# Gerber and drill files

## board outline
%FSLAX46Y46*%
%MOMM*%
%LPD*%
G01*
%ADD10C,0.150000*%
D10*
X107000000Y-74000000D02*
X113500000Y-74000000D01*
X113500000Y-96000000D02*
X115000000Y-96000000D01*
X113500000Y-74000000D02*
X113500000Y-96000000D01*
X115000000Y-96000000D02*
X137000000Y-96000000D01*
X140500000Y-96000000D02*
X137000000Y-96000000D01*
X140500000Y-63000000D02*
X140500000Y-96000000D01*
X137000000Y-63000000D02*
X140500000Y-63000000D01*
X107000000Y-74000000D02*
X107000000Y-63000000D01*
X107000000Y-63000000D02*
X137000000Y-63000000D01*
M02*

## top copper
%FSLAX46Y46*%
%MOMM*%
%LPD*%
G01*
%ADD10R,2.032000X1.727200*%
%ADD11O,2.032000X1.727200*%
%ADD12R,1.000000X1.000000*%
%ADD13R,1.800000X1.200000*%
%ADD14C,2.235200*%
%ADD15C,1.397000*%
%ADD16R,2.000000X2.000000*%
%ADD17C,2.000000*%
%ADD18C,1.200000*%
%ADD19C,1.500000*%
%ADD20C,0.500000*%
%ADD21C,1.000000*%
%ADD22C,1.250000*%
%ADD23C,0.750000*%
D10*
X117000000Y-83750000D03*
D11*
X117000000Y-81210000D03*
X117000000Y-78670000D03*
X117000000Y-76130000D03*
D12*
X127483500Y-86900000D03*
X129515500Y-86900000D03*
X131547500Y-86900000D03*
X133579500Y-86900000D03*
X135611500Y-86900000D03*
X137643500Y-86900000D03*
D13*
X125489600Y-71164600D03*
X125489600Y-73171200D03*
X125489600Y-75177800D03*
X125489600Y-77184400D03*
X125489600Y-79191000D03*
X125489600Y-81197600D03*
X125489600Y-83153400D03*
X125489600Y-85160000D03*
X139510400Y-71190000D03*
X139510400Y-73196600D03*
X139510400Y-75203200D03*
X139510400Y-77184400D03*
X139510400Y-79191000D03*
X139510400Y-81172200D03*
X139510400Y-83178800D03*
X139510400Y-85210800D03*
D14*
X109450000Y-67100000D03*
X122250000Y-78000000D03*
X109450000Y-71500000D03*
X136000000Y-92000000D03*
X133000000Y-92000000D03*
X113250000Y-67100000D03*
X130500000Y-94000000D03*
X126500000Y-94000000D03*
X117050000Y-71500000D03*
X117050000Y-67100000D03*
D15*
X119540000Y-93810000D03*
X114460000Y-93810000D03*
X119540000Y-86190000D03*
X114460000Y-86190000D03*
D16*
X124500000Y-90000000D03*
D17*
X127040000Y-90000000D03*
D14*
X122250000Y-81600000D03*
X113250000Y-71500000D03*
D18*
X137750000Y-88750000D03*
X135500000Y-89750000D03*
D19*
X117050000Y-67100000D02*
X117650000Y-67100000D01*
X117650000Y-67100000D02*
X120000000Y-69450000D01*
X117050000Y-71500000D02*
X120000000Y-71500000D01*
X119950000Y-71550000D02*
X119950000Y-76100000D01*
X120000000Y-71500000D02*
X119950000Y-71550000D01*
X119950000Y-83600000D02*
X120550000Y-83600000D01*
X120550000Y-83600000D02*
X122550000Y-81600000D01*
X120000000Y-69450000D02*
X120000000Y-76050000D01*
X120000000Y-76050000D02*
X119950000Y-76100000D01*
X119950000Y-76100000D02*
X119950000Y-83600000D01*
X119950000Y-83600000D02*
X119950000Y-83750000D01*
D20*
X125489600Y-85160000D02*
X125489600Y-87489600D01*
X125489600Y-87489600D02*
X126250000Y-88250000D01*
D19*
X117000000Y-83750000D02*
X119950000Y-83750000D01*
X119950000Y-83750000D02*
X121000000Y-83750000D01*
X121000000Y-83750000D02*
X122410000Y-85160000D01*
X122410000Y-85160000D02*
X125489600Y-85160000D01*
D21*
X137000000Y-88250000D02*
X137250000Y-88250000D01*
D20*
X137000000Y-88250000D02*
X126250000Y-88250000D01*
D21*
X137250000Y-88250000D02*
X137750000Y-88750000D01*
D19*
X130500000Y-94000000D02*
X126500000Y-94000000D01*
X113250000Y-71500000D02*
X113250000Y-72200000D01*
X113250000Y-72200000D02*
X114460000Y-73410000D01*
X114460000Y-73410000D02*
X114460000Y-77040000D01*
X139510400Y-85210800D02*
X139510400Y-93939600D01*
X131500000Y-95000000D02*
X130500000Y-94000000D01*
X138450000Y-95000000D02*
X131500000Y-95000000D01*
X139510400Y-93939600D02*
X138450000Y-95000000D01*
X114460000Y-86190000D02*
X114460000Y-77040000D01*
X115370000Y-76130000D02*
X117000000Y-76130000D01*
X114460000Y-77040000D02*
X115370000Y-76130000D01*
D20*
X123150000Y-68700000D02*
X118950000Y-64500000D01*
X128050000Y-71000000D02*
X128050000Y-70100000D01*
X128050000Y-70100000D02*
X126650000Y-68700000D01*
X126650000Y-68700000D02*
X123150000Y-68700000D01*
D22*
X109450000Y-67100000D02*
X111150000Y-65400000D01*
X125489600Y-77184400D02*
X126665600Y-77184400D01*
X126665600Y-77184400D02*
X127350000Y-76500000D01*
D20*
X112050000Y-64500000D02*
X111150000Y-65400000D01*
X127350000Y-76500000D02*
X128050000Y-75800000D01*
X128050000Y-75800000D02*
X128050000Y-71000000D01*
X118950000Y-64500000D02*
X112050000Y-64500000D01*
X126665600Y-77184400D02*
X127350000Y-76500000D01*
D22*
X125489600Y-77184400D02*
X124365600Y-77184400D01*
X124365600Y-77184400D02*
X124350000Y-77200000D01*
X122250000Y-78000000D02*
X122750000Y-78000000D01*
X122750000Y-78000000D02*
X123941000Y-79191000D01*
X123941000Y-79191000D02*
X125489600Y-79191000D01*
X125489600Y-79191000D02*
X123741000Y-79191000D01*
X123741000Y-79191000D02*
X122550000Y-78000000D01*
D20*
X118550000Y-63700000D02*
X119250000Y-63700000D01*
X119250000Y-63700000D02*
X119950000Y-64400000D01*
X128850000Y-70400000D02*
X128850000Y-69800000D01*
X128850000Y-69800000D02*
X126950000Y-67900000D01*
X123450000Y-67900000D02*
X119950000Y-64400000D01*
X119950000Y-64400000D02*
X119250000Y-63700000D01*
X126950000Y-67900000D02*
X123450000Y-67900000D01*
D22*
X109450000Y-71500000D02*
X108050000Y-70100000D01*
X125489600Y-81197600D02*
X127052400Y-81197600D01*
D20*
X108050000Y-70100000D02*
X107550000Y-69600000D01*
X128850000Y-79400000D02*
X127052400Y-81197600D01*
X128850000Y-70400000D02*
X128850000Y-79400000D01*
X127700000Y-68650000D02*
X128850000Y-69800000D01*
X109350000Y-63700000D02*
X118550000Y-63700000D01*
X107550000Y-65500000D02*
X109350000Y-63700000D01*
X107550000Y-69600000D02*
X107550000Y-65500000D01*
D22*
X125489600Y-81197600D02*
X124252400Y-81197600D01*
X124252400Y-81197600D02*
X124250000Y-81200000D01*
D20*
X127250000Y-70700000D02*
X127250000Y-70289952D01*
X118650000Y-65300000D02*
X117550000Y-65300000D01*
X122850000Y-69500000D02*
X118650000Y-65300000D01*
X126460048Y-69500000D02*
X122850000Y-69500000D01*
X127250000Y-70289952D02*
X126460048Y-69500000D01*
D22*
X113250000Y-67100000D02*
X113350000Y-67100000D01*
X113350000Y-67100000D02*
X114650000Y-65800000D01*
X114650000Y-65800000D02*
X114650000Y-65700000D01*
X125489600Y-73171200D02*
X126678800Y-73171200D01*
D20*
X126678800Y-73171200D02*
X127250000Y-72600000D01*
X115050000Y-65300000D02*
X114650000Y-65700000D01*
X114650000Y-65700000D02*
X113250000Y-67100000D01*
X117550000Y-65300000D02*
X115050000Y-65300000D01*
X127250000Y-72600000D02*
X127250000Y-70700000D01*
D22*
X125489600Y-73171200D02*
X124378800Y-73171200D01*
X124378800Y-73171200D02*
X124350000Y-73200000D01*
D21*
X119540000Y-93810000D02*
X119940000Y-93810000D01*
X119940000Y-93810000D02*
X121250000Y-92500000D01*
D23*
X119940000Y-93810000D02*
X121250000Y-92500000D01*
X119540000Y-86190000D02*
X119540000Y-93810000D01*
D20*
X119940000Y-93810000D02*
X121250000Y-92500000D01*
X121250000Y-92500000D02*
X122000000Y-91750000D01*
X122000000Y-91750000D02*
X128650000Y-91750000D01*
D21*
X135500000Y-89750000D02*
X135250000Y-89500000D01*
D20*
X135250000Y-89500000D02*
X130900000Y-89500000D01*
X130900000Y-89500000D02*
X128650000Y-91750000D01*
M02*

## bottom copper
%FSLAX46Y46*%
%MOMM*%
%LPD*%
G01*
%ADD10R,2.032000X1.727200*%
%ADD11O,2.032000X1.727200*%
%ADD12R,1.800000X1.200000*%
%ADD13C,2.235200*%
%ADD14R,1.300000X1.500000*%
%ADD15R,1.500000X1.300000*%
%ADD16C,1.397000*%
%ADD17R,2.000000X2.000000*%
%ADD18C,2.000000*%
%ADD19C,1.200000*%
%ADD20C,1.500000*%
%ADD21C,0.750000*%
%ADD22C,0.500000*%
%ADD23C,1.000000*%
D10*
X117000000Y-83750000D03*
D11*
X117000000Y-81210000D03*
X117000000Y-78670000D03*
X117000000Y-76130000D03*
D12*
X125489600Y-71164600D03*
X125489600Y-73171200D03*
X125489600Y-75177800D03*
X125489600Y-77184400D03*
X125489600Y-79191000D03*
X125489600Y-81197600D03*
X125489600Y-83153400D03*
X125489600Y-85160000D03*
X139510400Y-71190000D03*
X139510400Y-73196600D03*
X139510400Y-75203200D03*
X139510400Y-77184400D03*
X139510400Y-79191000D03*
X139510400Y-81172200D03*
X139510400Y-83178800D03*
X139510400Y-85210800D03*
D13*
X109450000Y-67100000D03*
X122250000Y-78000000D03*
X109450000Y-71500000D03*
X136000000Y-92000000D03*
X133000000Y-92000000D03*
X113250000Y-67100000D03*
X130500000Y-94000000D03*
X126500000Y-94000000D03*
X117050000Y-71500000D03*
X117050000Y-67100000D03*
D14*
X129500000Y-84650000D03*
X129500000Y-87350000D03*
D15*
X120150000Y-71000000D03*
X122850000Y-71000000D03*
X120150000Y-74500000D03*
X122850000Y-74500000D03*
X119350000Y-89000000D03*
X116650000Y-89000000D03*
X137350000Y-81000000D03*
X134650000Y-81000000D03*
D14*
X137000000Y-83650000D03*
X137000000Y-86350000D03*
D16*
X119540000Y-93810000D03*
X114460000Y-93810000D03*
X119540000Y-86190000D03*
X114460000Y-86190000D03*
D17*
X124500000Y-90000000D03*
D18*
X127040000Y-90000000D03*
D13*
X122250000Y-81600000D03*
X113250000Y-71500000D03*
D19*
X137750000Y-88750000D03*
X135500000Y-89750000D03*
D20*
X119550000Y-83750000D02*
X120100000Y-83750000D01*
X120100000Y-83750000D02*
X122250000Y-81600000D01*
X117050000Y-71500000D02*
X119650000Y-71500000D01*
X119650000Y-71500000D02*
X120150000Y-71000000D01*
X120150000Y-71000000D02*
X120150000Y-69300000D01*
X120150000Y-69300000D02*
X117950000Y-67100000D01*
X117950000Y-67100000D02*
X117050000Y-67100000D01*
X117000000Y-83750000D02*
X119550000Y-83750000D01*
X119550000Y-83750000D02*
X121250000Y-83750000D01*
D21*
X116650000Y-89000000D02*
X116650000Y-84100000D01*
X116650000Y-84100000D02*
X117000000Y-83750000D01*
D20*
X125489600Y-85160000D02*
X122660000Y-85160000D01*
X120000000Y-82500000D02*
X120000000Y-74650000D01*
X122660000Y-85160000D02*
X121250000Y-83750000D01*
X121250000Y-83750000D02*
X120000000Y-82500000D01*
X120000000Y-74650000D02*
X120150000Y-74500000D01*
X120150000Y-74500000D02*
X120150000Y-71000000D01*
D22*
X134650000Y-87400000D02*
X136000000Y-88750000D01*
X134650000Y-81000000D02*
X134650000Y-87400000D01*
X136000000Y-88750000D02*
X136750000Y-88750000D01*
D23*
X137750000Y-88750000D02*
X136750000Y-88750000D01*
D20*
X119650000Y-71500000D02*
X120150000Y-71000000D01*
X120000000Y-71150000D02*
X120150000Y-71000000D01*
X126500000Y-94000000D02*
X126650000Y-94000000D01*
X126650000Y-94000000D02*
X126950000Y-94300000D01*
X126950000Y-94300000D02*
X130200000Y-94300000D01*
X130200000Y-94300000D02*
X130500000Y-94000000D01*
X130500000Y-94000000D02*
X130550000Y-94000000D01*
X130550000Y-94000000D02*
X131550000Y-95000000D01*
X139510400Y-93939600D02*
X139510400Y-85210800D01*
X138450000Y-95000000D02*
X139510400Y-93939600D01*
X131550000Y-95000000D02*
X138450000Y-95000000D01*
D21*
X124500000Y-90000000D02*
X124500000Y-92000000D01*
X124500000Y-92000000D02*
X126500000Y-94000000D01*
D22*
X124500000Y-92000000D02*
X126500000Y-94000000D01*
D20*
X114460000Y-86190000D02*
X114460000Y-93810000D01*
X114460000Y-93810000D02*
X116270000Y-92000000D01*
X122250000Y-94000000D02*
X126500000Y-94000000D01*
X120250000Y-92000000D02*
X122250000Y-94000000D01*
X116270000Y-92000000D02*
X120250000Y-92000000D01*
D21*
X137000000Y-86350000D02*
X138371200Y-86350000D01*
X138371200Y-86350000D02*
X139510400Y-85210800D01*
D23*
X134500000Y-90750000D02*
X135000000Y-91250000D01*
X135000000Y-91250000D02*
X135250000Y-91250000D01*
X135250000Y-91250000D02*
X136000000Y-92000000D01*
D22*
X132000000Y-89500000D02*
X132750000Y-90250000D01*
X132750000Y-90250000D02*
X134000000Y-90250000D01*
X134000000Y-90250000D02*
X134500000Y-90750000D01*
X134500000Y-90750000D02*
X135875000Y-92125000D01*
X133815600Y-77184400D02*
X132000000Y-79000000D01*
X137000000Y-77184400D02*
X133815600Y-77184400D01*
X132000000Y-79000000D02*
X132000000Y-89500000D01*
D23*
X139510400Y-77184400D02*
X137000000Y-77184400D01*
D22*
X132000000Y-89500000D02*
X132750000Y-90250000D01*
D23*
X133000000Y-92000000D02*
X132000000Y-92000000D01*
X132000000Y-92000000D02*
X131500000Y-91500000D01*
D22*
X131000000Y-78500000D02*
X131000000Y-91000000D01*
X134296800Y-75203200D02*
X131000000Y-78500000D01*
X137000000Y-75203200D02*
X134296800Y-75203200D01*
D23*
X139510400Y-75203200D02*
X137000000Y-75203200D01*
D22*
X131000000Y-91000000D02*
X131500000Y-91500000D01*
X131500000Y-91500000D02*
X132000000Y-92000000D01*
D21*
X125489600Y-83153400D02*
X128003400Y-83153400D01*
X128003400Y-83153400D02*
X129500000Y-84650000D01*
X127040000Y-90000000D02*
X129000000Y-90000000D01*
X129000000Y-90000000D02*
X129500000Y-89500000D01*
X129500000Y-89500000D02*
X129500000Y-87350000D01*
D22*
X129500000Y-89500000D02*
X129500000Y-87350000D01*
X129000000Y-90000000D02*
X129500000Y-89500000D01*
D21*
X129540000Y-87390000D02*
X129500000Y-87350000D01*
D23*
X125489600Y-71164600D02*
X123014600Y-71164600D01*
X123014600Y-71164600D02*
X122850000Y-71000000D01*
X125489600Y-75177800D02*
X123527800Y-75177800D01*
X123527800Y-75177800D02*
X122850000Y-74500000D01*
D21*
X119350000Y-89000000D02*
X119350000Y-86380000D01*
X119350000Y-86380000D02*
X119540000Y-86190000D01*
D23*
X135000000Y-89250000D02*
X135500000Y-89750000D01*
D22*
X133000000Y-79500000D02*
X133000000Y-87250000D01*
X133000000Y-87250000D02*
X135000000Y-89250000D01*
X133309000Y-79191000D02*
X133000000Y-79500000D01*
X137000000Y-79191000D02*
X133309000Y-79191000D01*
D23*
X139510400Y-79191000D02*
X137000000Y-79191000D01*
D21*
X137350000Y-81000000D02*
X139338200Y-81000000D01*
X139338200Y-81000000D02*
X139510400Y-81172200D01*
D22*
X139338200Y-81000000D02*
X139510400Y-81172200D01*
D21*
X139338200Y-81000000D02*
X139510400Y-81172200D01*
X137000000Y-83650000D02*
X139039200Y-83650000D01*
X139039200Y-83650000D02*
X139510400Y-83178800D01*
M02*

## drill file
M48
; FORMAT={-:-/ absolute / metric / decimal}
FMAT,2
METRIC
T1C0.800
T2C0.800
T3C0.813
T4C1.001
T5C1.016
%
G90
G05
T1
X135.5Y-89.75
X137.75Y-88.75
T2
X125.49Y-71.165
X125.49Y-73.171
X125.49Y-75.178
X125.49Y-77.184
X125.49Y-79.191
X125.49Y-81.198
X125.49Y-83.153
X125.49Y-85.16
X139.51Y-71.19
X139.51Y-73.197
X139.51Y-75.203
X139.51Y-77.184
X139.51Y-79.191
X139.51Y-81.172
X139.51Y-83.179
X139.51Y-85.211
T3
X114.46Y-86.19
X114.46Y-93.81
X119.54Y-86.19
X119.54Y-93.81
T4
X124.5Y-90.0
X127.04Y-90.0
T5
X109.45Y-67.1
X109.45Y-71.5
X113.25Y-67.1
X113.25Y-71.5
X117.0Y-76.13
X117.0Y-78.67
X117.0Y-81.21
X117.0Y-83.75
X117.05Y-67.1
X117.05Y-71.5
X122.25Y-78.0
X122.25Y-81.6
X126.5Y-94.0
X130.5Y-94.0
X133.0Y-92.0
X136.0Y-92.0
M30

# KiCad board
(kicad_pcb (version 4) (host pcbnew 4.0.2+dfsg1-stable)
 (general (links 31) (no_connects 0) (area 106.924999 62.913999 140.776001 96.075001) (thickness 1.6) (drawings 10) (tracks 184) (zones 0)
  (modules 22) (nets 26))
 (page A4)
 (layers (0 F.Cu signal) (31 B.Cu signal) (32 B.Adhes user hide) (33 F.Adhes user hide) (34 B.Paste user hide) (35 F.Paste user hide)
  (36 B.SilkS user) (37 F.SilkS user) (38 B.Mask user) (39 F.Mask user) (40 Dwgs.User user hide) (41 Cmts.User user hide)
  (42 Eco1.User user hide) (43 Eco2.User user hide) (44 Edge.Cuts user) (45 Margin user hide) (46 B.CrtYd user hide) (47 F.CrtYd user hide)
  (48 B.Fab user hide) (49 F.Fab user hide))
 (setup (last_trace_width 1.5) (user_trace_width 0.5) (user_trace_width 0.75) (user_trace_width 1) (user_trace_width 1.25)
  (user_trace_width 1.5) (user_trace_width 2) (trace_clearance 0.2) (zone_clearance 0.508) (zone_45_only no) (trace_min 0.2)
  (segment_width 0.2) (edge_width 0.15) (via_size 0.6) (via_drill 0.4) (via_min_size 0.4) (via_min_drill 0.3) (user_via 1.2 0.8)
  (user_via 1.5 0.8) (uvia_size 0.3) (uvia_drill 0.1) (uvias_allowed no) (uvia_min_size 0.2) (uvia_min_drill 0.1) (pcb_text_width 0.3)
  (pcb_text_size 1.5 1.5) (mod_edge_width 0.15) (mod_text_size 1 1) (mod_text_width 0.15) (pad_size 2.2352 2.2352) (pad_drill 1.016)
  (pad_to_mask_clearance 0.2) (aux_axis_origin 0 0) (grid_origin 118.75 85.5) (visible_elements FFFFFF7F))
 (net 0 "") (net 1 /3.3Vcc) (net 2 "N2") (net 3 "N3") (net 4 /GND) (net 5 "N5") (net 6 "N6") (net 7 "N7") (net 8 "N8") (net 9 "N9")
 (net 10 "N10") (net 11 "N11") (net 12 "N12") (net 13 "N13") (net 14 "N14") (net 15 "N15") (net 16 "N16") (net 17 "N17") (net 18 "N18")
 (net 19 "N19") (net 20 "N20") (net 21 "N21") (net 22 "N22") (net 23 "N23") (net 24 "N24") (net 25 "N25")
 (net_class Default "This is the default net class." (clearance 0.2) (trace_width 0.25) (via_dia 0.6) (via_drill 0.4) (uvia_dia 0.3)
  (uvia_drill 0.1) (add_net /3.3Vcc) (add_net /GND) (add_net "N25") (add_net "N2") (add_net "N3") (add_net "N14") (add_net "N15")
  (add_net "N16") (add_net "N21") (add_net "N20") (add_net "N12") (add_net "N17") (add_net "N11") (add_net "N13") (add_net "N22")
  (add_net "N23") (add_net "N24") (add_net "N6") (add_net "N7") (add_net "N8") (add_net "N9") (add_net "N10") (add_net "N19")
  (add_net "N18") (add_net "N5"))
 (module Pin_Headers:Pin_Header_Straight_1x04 (layer F.Cu) (at 117 83.75 180)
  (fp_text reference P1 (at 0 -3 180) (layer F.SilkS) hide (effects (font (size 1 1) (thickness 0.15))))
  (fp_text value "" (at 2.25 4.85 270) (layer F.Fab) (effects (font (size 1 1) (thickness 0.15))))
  (pad 1 thru_hole rect (at 0 0 180) (size 2.032 1.7272) (drill 1.016) (layers *.Cu *.Mask F.SilkS) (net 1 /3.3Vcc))
  (pad 2 thru_hole oval (at 0 2.54 180) (size 2.032 1.7272) (drill 1.016) (layers *.Cu *.Mask F.SilkS) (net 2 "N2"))
  (pad 3 thru_hole oval (at 0 5.08 180) (size 2.032 1.7272) (drill 1.016) (layers *.Cu *.Mask F.SilkS) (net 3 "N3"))
  (pad 4 thru_hole oval (at 0 7.62 180) (size 2.032 1.7272) (drill 1.016) (layers *.Cu *.Mask F.SilkS) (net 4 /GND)))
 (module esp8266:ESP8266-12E (layer F.Cu) (at 132.5 75)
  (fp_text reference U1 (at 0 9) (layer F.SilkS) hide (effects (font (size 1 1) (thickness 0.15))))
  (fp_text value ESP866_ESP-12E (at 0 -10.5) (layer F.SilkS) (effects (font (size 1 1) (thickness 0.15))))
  (pad 9 smd rect (at -5.0165 11.9 90) (size 1 1) (layers F.Cu F.Paste F.Mask) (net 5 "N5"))
  (pad 10 smd rect (at -2.9845 11.9 90) (size 1 1) (layers F.Cu F.Paste F.Mask) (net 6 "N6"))
  (pad 11 smd rect (at -0.9525 11.9 90) (size 1 1) (layers F.Cu F.Paste F.Mask) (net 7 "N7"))
  (pad 12 smd rect (at 1.0795 11.9 90) (size 1 1) (layers F.Cu F.Paste F.Mask) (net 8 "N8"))
  (pad 13 smd rect (at 3.1115 11.9 90) (size 1 1) (layers F.Cu F.Paste F.Mask) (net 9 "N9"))
  (pad 14 smd rect (at 5.1435 11.9 90) (size 1 1) (layers F.Cu F.Paste F.Mask) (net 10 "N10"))
  (pad 1 thru_hole rect (at -7.0104 -3.8354) (size 1.8 1.2) (drill 0.8) (layers *.Cu *.Mask F.SilkS) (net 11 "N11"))
  (pad 2 thru_hole rect (at -7.0104 -1.8288) (size 1.8 1.2) (drill 0.8) (layers *.Cu *.Mask F.SilkS) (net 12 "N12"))
  (pad 3 thru_hole rect (at -7.0104 0.1778) (size 1.8 1.2) (drill 0.8) (layers *.Cu *.Mask F.SilkS) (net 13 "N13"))
  (pad 4 thru_hole rect (at -7.0104 2.1844) (size 1.8 1.2) (drill 0.8) (layers *.Cu *.Mask F.SilkS) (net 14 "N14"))
  (pad 5 thru_hole rect (at -7.0104 4.191) (size 1.8 1.2) (drill 0.8) (layers *.Cu *.Mask F.SilkS) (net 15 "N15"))
  (pad 6 thru_hole rect (at -7.0104 6.1976) (size 1.8 1.2) (drill 0.8) (layers *.Cu *.Mask F.SilkS) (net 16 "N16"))
  (pad 7 thru_hole rect (at -7.0104 8.1534) (size 1.8 1.2) (drill 0.8) (layers *.Cu *.Mask F.SilkS) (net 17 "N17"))
  (pad 8 thru_hole rect (at -7.0104 10.16) (size 1.8 1.2) (drill 0.8) (layers *.Cu *.Mask F.SilkS) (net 1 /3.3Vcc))
  (pad 22 thru_hole rect (at 7.0104 -3.81) (size 1.8 1.2) (drill 0.8) (layers *.Cu *.Mask F.SilkS) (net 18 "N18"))
  (pad 21 thru_hole rect (at 7.0104 -1.8034) (size 1.8 1.2) (drill 0.8) (layers *.Cu *.Mask F.SilkS) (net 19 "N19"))
  (pad 20 thru_hole rect (at 7.0104 0.2032) (size 1.8 1.2) (drill 0.8) (layers *.Cu *.Mask F.SilkS) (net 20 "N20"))
  (pad 19 thru_hole rect (at 7.0104 2.1844) (size 1.8 1.2) (drill 0.8) (layers *.Cu *.Mask F.SilkS) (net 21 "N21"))
  (pad 18 thru_hole rect (at 7.0104 4.191) (size 1.8 1.2) (drill 0.8) (layers *.Cu *.Mask F.SilkS) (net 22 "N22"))
  (pad 17 thru_hole rect (at 7.0104 6.1722) (size 1.8 1.2) (drill 0.8) (layers *.Cu *.Mask F.SilkS) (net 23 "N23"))
  (pad 16 thru_hole rect (at 7.0104 8.1788) (size 1.8 1.2) (drill 0.8) (layers *.Cu *.Mask F.SilkS) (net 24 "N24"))
  (pad 15 thru_hole rect (at 7.0104 10.2108) (size 1.8 1.2) (drill 0.8) (layers *.Cu *.Mask F.SilkS) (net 4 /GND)))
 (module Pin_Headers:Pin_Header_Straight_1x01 (layer F.Cu) (at 109.45 67.1)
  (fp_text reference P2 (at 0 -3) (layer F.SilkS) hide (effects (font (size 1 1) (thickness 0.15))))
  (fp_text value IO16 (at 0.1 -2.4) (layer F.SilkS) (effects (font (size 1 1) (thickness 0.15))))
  (pad 1 thru_hole circle (at 0 0) (size 2.2352 2.2352) (drill 1.016) (layers *.Cu *.Mask F.SilkS) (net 14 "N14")))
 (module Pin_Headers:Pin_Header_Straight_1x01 (layer F.Cu) (at 122.25 78)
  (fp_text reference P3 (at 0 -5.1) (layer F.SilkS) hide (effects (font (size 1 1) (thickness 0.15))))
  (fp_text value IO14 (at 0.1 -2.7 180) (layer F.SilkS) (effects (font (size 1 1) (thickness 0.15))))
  (pad 1 thru_hole circle (at 0 0) (size 2.2352 2.2352) (drill 1.016) (layers *.Cu *.Mask F.SilkS) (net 15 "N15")))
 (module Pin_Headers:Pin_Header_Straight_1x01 (layer F.Cu) (at 109.45 71.5)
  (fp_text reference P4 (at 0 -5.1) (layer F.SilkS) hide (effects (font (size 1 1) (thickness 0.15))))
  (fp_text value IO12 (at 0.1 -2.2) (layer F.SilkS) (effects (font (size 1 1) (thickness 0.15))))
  (pad 1 thru_hole circle (at 0 0) (size 2.2352 2.2352) (drill 1.016) (layers *.Cu *.Mask F.SilkS) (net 16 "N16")))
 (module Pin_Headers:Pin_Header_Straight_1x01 (layer F.Cu) (at 136 92)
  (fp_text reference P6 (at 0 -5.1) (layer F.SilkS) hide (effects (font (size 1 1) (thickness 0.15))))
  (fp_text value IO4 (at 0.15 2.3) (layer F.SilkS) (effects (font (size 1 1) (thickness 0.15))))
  (pad 1 thru_hole circle (at 0 0) (size 2.2352 2.2352) (drill 1.016) (layers *.Cu *.Mask F.SilkS) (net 21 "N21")))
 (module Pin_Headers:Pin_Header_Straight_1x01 (layer F.Cu) (at 133 92)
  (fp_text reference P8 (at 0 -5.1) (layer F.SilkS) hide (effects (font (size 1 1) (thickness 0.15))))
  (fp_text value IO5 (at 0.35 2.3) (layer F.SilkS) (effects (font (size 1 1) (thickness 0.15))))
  (pad 1 thru_hole circle (at 0 0) (size 2.2352 2.2352) (drill 1.016) (layers *.Cu *.Mask F.SilkS) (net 20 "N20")))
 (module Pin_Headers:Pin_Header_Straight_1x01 (layer F.Cu) (at 113.25 67.1)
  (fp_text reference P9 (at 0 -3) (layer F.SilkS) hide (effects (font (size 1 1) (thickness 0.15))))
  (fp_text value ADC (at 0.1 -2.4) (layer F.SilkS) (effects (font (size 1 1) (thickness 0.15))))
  (pad 1 thru_hole circle (at 0 0) (size 2.2352 2.2352) (drill 1.016) (layers *.Cu *.Mask F.SilkS) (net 12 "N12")))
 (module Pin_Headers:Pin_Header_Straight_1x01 (layer F.Cu) (at 130.5 94)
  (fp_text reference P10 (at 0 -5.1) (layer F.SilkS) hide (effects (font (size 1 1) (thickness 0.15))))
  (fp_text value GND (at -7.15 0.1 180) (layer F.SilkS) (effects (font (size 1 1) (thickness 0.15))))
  (pad 1 thru_hole circle (at 0 0) (size 2.2352 2.2352) (drill 1.016) (layers *.Cu *.Mask F.SilkS) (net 4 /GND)))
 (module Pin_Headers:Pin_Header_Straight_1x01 (layer F.Cu) (at 126.5 94)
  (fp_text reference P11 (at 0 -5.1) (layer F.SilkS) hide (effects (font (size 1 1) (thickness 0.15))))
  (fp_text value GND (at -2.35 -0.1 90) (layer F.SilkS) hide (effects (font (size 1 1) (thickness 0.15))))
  (pad 1 thru_hole circle (at 0 0) (size 2.2352 2.2352) (drill 1.016) (layers *.Cu *.Mask F.SilkS) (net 4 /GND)))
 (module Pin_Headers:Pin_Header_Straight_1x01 (layer F.Cu) (at 117.05 71.5)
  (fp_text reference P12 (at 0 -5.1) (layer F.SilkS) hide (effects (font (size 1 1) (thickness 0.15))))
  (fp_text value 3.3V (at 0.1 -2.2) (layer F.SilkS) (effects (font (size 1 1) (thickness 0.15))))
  (pad 1 thru_hole circle (at 0 0) (size 2.2352 2.2352) (drill 1.016) (layers *.Cu *.Mask F.SilkS) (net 1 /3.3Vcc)))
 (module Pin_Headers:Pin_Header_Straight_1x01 (layer F.Cu) (at 117.05 67.1)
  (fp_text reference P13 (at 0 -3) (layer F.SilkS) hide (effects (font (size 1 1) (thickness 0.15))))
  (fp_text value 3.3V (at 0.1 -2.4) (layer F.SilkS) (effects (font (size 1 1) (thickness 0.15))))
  (pad 1 thru_hole circle (at 0 0) (size 2.2352 2.2352) (drill 1.016) (layers *.Cu *.Mask F.SilkS) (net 1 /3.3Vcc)))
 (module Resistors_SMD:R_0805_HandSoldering (layer B.Cu) (at 129.5 86 270)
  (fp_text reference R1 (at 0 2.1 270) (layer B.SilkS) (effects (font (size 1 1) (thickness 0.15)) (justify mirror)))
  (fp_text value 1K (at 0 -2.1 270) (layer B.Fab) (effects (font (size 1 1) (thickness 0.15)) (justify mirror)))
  (pad 1 smd rect (at -1.35 0 270) (size 1.5 1.3) (layers B.Cu B.Paste B.Mask) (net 17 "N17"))
  (pad 2 smd rect (at 1.35 0 270) (size 1.5 1.3) (layers B.Cu B.Paste B.Mask) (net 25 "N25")))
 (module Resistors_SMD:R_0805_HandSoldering (layer B.Cu) (at 121.5 71)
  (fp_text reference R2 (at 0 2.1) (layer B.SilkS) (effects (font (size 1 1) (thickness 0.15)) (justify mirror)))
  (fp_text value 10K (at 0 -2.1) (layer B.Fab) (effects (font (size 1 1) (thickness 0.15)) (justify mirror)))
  (pad 1 smd rect (at -1.35 0) (size 1.5 1.3) (layers B.Cu B.Paste B.Mask) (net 1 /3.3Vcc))
  (pad 2 smd rect (at 1.35 0) (size 1.5 1.3) (layers B.Cu B.Paste B.Mask) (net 11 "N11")))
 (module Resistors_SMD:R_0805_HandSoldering (layer B.Cu) (at 121.5 74.5)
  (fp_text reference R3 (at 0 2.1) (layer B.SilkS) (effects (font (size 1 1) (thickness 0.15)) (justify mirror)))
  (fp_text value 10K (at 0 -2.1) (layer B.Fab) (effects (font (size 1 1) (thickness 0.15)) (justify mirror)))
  (pad 1 smd rect (at -1.35 0) (size 1.5 1.3) (layers B.Cu B.Paste B.Mask) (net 1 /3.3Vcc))
  (pad 2 smd rect (at 1.35 0) (size 1.5 1.3) (layers B.Cu B.Paste B.Mask) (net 13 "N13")))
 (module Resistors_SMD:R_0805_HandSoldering (layer B.Cu) (at 118 89 180)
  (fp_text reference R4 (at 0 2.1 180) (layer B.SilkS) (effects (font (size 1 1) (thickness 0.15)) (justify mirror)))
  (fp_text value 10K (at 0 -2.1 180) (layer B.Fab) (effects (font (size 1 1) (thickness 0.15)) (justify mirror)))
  (pad 1 smd rect (at -1.35 0 180) (size 1.5 1.3) (layers B.Cu B.Paste B.Mask) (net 22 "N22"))
  (pad 2 smd rect (at 1.35 0 180) (size 1.5 1.3) (layers B.Cu B.Paste B.Mask) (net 1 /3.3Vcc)))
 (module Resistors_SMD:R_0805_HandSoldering (layer B.Cu) (at 136 81 180)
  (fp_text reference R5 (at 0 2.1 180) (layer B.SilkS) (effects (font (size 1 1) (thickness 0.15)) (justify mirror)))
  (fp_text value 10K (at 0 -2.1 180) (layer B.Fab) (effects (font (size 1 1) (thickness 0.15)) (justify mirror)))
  (pad 1 smd rect (at -1.35 0 180) (size 1.5 1.3) (layers B.Cu B.Paste B.Mask) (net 23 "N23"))
  (pad 2 smd rect (at 1.35 0 180) (size 1.5 1.3) (layers B.Cu B.Paste B.Mask) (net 1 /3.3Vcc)))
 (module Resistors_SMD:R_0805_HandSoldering (layer B.Cu) (at 137 85 270)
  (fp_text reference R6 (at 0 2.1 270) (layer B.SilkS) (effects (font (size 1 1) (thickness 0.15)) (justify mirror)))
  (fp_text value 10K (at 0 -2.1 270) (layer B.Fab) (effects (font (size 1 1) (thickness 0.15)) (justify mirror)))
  (pad 1 smd rect (at -1.35 0 270) (size 1.5 1.3) (layers B.Cu B.Paste B.Mask) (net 24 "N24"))
  (pad 2 smd rect (at 1.35 0 270) (size 1.5 1.3) (layers B.Cu B.Paste B.Mask) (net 4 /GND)))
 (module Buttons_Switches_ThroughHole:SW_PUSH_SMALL (layer F.Cu) (at 117 90 270)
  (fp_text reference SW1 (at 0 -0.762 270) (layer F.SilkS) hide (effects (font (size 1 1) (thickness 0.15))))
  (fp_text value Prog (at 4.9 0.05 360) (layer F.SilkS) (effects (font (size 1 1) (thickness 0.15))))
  (pad 1 thru_hole circle (at 3.81 -2.54 270) (size 1.397 1.397) (drill 0.8128) (layers *.Cu *.Mask F.SilkS) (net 22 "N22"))
  (pad 2 thru_hole circle (at 3.81 2.54 270) (size 1.397 1.397) (drill 0.8128) (layers *.Cu *.Mask F.SilkS) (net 4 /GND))
  (pad 1 thru_hole circle (at -3.81 -2.54 270) (size 1.397 1.397) (drill 0.8128) (layers *.Cu *.Mask F.SilkS) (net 22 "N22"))
  (pad 2 thru_hole circle (at -3.81 2.54 270) (size 1.397 1.397) (drill 0.8128) (layers *.Cu *.Mask F.SilkS) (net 4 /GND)))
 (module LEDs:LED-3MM (layer F.Cu) (at 124.5 90)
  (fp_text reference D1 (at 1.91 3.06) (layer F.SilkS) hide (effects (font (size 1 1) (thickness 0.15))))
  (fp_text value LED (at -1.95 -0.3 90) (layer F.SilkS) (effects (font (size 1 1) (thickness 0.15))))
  (pad 1 thru_hole rect (at 0 0 90) (size 2 2) (drill 1.00076) (layers *.Cu *.Mask F.SilkS) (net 4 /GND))
  (pad 2 thru_hole circle (at 2.54 0) (size 2 2) (drill 1.00076) (layers *.Cu *.Mask F.SilkS) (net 25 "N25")))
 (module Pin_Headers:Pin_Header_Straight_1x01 (layer F.Cu) (at 122.25 81.6)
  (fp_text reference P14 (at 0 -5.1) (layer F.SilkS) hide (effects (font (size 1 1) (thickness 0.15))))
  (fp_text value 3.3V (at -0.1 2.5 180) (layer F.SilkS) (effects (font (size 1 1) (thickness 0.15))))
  (pad 1 thru_hole circle (at 0 0) (size 2.2352 2.2352) (drill 1.016) (layers *.Cu *.Mask F.SilkS) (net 1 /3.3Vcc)))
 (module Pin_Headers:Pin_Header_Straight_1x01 (layer F.Cu) (at 113.25 71.5)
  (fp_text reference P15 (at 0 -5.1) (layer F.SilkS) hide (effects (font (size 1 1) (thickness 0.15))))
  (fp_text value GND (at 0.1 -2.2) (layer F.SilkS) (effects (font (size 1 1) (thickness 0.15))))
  (pad 1 thru_hole circle (at 0 0) (size 2.2352 2.2352) (drill 1.016) (layers *.Cu *.Mask F.SilkS) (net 4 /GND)))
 (gr_line (start 107 74) (end 113.5 74) (angle 90) (layer Edge.Cuts) (width 0.15))
 (gr_line (start 113.5 96) (end 115 96) (angle 90) (layer Edge.Cuts) (width 0.15))
 (gr_line (start 113.5 74) (end 113.5 96) (angle 90) (layer Edge.Cuts) (width 0.15))
 (gr_line (start 115 96) (end 137 96) (angle 90) (layer Edge.Cuts) (width 0.15))
 (gr_line (start 140.5 96) (end 137 96) (angle 90) (layer Edge.Cuts) (width 0.15))
 (gr_line (start 140.5 63) (end 140.5 96) (angle 90) (layer Edge.Cuts) (width 0.15))
 (gr_line (start 137 63) (end 140.5 63) (angle 90) (layer Edge.Cuts) (width 0.15))
 (gr_line (start 107 74) (end 107 63) (angle 90) (layer Edge.Cuts) (width 0.15))
 (gr_line (start 107 63) (end 137 63) (angle 90) (layer Edge.Cuts) (width 0.15))
 (segment (start 119.55 83.75) (end 120.1 83.75) (width 1.5) (layer B.Cu) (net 1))
 (segment (start 120.1 83.75) (end 122.25 81.6) (width 1.5) (layer B.Cu) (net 1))
 (segment (start 117.05 71.5) (end 119.65 71.5) (width 1.5) (layer B.Cu) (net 1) (status 30))
 (segment (start 119.65 71.5) (end 120.15 71) (width 1.5) (layer B.Cu) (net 1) (status 30))
 (segment (start 120.15 71) (end 120.15 69.3) (width 1.5) (layer B.Cu) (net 1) (status 10))
 (segment (start 120.15 69.3) (end 117.95 67.1) (width 1.5) (layer B.Cu) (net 1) (status 20))
 (segment (start 117.95 67.1) (end 117.05 67.1) (width 1.5) (layer B.Cu) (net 1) (status 30))
 (segment (start 117.05 67.1) (end 117.65 67.1) (width 1.5) (layer F.Cu) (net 1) (status 30))
 (segment (start 117.65 67.1) (end 120 69.45) (width 1.5) (layer F.Cu) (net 1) (status 10))
 (segment (start 117.05 71.5) (end 120 71.5) (width 1.5) (layer F.Cu) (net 1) (status 10))
 (segment (start 119.95 71.55) (end 119.95 76.1) (width 1.5) (layer F.Cu) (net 1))
 (segment (start 120 71.5) (end 119.95 71.55) (width 1.5) (layer F.Cu) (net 1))
 (segment (start 119.95 83.6) (end 120.55 83.6) (width 1.5) (layer F.Cu) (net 1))
 (segment (start 120.55 83.6) (end 122.55 81.6) (width 1.5) (layer F.Cu) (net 1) (status 20))
 (segment (start 117 83.75) (end 119.55 83.75) (width 1.5) (layer B.Cu) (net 1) (status 10))
 (segment (start 119.55 83.75) (end 121.25 83.75) (width 1.5) (layer B.Cu) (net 1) (status 10))
 (segment (start 120 69.45) (end 120 76.05) (width 1.5) (layer F.Cu) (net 1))
 (segment (start 120 76.05) (end 119.95 76.1) (width 1.5) (layer F.Cu) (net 1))
 (segment (start 119.95 76.1) (end 119.95 83.6) (width 1.5) (layer F.Cu) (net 1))
 (segment (start 119.95 83.6) (end 119.95 83.75) (width 1.5) (layer F.Cu) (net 1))
 (segment (start 116.65 89) (end 116.65 84.1) (width 0.75) (layer B.Cu) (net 1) (status 30))
 (segment (start 116.65 84.1) (end 117 83.75) (width 0.75) (layer B.Cu) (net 1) (status 30))
 (segment (start 125.4896 85.16) (end 122.66 85.16) (width 1.5) (layer B.Cu) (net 1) (status 10))
 (segment (start 120 82.5) (end 120 74.65) (width 1.5) (layer B.Cu) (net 1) (status 20))
 (segment (start 122.66 85.16) (end 121.25 83.75) (width 1.5) (layer B.Cu) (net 1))
 (segment (start 121.25 83.75) (end 120 82.5) (width 1.5) (layer B.Cu) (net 1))
 (segment (start 120 74.65) (end 120.15 74.5) (width 1.5) (layer B.Cu) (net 1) (status 30))
 (segment (start 120.15 74.5) (end 120.15 71) (width 1.5) (layer B.Cu) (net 1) (status 30))
 (segment (start 125.4896 85.16) (end 125.4896 87.4896) (width 0.5) (layer F.Cu) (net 1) (status 10))
 (segment (start 125.4896 87.4896) (end 126.25 88.25) (width 0.5) (layer F.Cu) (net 1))
 (segment (start 117 83.75) (end 119.95 83.75) (width 1.5) (layer F.Cu) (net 1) (status 10))
 (segment (start 119.95 83.75) (end 121 83.75) (width 1.5) (layer F.Cu) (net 1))
 (segment (start 121 83.75) (end 122.41 85.16) (width 1.5) (layer F.Cu) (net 1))
 (segment (start 122.41 85.16) (end 125.4896 85.16) (width 1.5) (layer F.Cu) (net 1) (status 20))
 (segment (start 137 88.25) (end 137.25 88.25) (width 1) (layer F.Cu) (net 1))
 (segment (start 137 88.25) (end 126.25 88.25) (width 0.5) (layer F.Cu) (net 1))
 (segment (start 134.65 87.4) (end 136 88.75) (width 0.5) (layer B.Cu) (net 1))
 (segment (start 134.65 81) (end 134.65 87.4) (width 0.5) (layer B.Cu) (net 1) (status 10))
 (segment (start 136 88.75) (end 136.75 88.75) (width 0.5) (layer B.Cu) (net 1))
 (via (at 137.75 88.75) (size 1.2) (drill 0.8) (layers F.Cu B.Cu) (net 1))
 (segment (start 137.75 88.75) (end 136.75 88.75) (width 1) (layer B.Cu) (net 1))
 (segment (start 137.25 88.25) (end 137.75 88.75) (width 1) (layer F.Cu) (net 1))
 (segment (start 119.65 71.5) (end 120.15 71) (width 1.5) (layer B.Cu) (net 1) (status 30))
 (segment (start 120 71.15) (end 120.15 71) (width 1.5) (layer B.Cu) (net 1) (status 30))
 (segment (start 126.5 94) (end 126.65 94) (width 1.5) (layer B.Cu) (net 4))
 (segment (start 126.65 94) (end 126.95 94.3) (width 1.5) (layer B.Cu) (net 4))
 (segment (start 126.95 94.3) (end 130.2 94.3) (width 1.5) (layer B.Cu) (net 4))
 (segment (start 130.2 94.3) (end 130.5 94) (width 1.5) (layer B.Cu) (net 4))
 (segment (start 130.5 94) (end 126.5 94) (width 1.5) (layer F.Cu) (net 4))
 (segment (start 113.25 71.5) (end 113.25 72.2) (width 1.5) (layer F.Cu) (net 4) (status 30))
 (segment (start 113.25 72.2) (end 114.46 73.41) (width 1.5) (layer F.Cu) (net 4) (status 10))
 (segment (start 114.46 73.41) (end 114.46 77.04) (width 1.5) (layer F.Cu) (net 4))
 (segment (start 130.5 94) (end 130.55 94) (width 1.5) (layer B.Cu) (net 4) (status 30))
 (segment (start 130.55 94) (end 131.55 95) (width 1.5) (layer B.Cu) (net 4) (status 10))
 (segment (start 139.5104 93.9396) (end 139.5104 85.2108) (width 1.5) (layer B.Cu) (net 4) (status 20))
 (segment (start 138.45 95) (end 139.5104 93.9396) (width 1.5) (layer B.Cu) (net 4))
 (segment (start 131.55 95) (end 138.45 95) (width 1.5) (layer B.Cu) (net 4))
 (segment (start 139.5104 85.2108) (end 139.5104 93.9396) (width 1.5) (layer F.Cu) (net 4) (status 10))
 (segment (start 131.5 95) (end 130.5 94) (width 1.5) (layer F.Cu) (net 4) (status 20))
 (segment (start 138.45 95) (end 131.5 95) (width 1.5) (layer F.Cu) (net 4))
 (segment (start 139.5104 93.9396) (end 138.45 95) (width 1.5) (layer F.Cu) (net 4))
 (segment (start 124.5 90) (end 124.5 92) (width 0.75) (layer B.Cu) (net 4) (status 10))
 (segment (start 124.5 92) (end 126.5 94) (width 0.75) (layer B.Cu) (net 4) (status 20))
 (segment (start 124.5 92) (end 126.5 94) (width 0.5) (layer B.Cu) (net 4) (status 20))
 (segment (start 114.46 86.19) (end 114.46 93.81) (width 1.5) (layer B.Cu) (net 4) (status 30))
 (segment (start 114.46 93.81) (end 116.27 92) (width 1.5) (layer B.Cu) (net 4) (status 10))
 (segment (start 122.25 94) (end 126.5 94) (width 1.5) (layer B.Cu) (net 4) (status 20))
 (segment (start 120.25 92) (end 122.25 94) (width 1.5) (layer B.Cu) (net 4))
 (segment (start 116.27 92) (end 120.25 92) (width 1.5) (layer B.Cu) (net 4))
 (segment (start 114.46 86.19) (end 114.46 77.04) (width 1.5) (layer F.Cu) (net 4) (status 10))
 (segment (start 115.37 76.13) (end 117 76.13) (width 1.5) (layer F.Cu) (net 4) (status 20))
 (segment (start 114.46 77.04) (end 115.37 76.13) (width 1.5) (layer F.Cu) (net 4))
 (segment (start 137 86.35) (end 138.3712 86.35) (width 0.75) (layer B.Cu) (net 4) (status 10))
 (segment (start 138.3712 86.35) (end 139.5104 85.2108) (width 0.75) (layer B.Cu) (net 4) (status 20))
 (segment (start 123.15 68.7) (end 118.95 64.5) (width 0.5) (layer F.Cu) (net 14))
 (segment (start 128.05 71) (end 128.05 70.1) (width 0.5) (layer F.Cu) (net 14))
 (segment (start 128.05 70.1) (end 126.65 68.7) (width 0.5) (layer F.Cu) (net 14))
 (segment (start 126.65 68.7) (end 123.15 68.7) (width 0.5) (layer F.Cu) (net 14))
 (segment (start 109.45 67.1) (end 111.15 65.4) (width 1.25) (layer F.Cu) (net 14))
 (segment (start 125.4896 77.1844) (end 126.6656 77.1844) (width 1.25) (layer F.Cu) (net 14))
 (segment (start 126.6656 77.1844) (end 127.35 76.5) (width 1.25) (layer F.Cu) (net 14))
 (segment (start 112.05 64.5) (end 111.15 65.4) (width 0.5) (layer F.Cu) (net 14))
 (segment (start 127.35 76.5) (end 128.05 75.8) (width 0.5) (layer F.Cu) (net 14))
 (segment (start 128.05 75.8) (end 128.05 71) (width 0.5) (layer F.Cu) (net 14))
 (segment (start 118.95 64.5) (end 112.05 64.5) (width 0.5) (layer F.Cu) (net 14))
 (segment (start 126.6656 77.1844) (end 127.35 76.5) (width 0.5) (layer F.Cu) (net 14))
 (segment (start 125.4896 77.1844) (end 124.3656 77.1844) (width 1.25) (layer F.Cu) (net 14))
 (segment (start 124.3656 77.1844) (end 124.35 77.2) (width 1.25) (layer F.Cu) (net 14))
 (segment (start 122.25 78) (end 122.75 78) (width 1.25) (layer F.Cu) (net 15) (status 30))
 (segment (start 122.75 78) (end 123.941 79.191) (width 1.25) (layer F.Cu) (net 15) (status 10))
 (segment (start 123.941 79.191) (end 125.4896 79.191) (width 1.25) (layer F.Cu) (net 15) (status 20))
 (segment (start 125.4896 79.191) (end 123.741 79.191) (width 1.25) (layer F.Cu) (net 15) (status 10))
 (segment (start 123.741 79.191) (end 122.55 78) (width 1.25) (layer F.Cu) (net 15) (status 20))
 (segment (start 118.55 63.7) (end 119.25 63.7) (width 0.5) (layer F.Cu) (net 16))
 (segment (start 119.25 63.7) (end 119.95 64.4) (width 0.5) (layer F.Cu) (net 16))
 (segment (start 128.85 70.4) (end 128.85 69.8) (width 0.5) (layer F.Cu) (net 16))
 (segment (start 128.85 69.8) (end 126.95 67.9) (width 0.5) (layer F.Cu) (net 16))
 (segment (start 123.45 67.9) (end 119.95 64.4) (width 0.5) (layer F.Cu) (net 16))
 (segment (start 119.95 64.4) (end 119.25 63.7) (width 0.5) (layer F.Cu) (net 16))
 (segment (start 126.95 67.9) (end 123.45 67.9) (width 0.5) (layer F.Cu) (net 16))
 (segment (start 109.45 71.5) (end 108.05 70.1) (width 1.25) (layer F.Cu) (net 16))
 (segment (start 125.4896 81.1976) (end 127.0524 81.1976) (width 1.25) (layer F.Cu) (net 16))
 (segment (start 108.05 70.1) (end 107.55 69.6) (width 0.5) (layer F.Cu) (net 16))
 (segment (start 128.85 79.4) (end 127.0524 81.1976) (width 0.5) (layer F.Cu) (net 16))
 (segment (start 128.85 70.4) (end 128.85 79.4) (width 0.5) (layer F.Cu) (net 16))
 (segment (start 127.7 68.65) (end 128.85 69.8) (width 0.5) (layer F.Cu) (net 16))
 (segment (start 109.35 63.7) (end 118.55 63.7) (width 0.5) (layer F.Cu) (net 16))
 (segment (start 107.55 65.5) (end 109.35 63.7) (width 0.5) (layer F.Cu) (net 16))
 (segment (start 107.55 69.6) (end 107.55 65.5) (width 0.5) (layer F.Cu) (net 16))
 (segment (start 125.4896 81.1976) (end 124.2524 81.1976) (width 1.25) (layer F.Cu) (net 16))
 (segment (start 124.2524 81.1976) (end 124.25 81.2) (width 1.25) (layer F.Cu) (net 16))
 (segment (start 134.5 90.75) (end 135 91.25) (width 1) (layer B.Cu) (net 21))
 (segment (start 135 91.25) (end 135.25 91.25) (width 1) (layer B.Cu) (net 21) (status 20))
 (segment (start 135.25 91.25) (end 136 92) (width 1) (layer B.Cu) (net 21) (status 30))
 (segment (start 132 89.5) (end 132.75 90.25) (width 0.5) (layer B.Cu) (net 21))
 (segment (start 132.75 90.25) (end 134 90.25) (width 0.5) (layer B.Cu) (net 21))
 (segment (start 134 90.25) (end 134.5 90.75) (width 0.5) (layer B.Cu) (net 21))
 (segment (start 134.5 90.75) (end 135.875 92.125) (width 0.5) (layer B.Cu) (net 21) (status 20))
 (segment (start 133.8156 77.1844) (end 132 79) (width 0.5) (layer B.Cu) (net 21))
 (segment (start 137 77.1844) (end 133.8156 77.1844) (width 0.5) (layer B.Cu) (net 21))
 (segment (start 132 79) (end 132 89.5) (width 0.5) (layer B.Cu) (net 21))
 (segment (start 139.5104 77.1844) (end 137 77.1844) (width 1) (layer B.Cu) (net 21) (status 10))
 (segment (start 132 89.5) (end 132.75 90.25) (width 0.5) (layer B.Cu) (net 21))
 (segment (start 133 92) (end 132 92) (width 1) (layer B.Cu) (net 20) (status 30))
 (segment (start 132 92) (end 131.5 91.5) (width 1) (layer B.Cu) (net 20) (status 10))
 (segment (start 131 78.5) (end 131 91) (width 0.5) (layer B.Cu) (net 20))
 (segment (start 134.2968 75.2032) (end 131 78.5) (width 0.5) (layer B.Cu) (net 20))
 (segment (start 137 75.2032) (end 134.2968 75.2032) (width 0.5) (layer B.Cu) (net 20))
 (segment (start 139.5104 75.2032) (end 137 75.2032) (width 1) (layer B.Cu) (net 20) (status 10))
 (segment (start 131 91) (end 131.5 91.5) (width 0.5) (layer B.Cu) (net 20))
 (segment (start 131.5 91.5) (end 132 92) (width 0.5) (layer B.Cu) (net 20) (status 20))
 (segment (start 127.25 70.7) (end 127.25 70.289952) (width 0.5) (layer F.Cu) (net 12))
 (segment (start 118.65 65.3) (end 117.55 65.3) (width 0.5) (layer F.Cu) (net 12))
 (segment (start 122.85 69.5) (end 118.65 65.3) (width 0.5) (layer F.Cu) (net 12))
 (segment (start 126.460048 69.5) (end 122.85 69.5) (width 0.5) (layer F.Cu) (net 12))
 (segment (start 127.25 70.289952) (end 126.460048 69.5) (width 0.5) (layer F.Cu) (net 12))
 (segment (start 113.25 67.1) (end 113.35 67.1) (width 1.25) (layer F.Cu) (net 12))
 (segment (start 113.35 67.1) (end 114.65 65.8) (width 1.25) (layer F.Cu) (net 12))
 (segment (start 114.65 65.8) (end 114.65 65.7) (width 1.25) (layer F.Cu) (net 12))
 (segment (start 125.4896 73.1712) (end 126.6788 73.1712) (width 1.25) (layer F.Cu) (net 12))
 (segment (start 126.6788 73.1712) (end 127.25 72.6) (width 0.5) (layer F.Cu) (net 12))
 (segment (start 115.05 65.3) (end 114.65 65.7) (width 0.5) (layer F.Cu) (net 12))
 (segment (start 114.65 65.7) (end 113.25 67.1) (width 0.5) (layer F.Cu) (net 12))
 (segment (start 117.55 65.3) (end 115.05 65.3) (width 0.5) (layer F.Cu) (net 12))
 (segment (start 127.25 72.6) (end 127.25 70.7) (width 0.5) (layer F.Cu) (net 12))
 (segment (start 125.4896 73.1712) (end 124.3788 73.1712) (width 1.25) (layer F.Cu) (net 12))
 (segment (start 124.3788 73.1712) (end 124.35 73.2) (width 1.25) (layer F.Cu) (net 12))
 (segment (start 125.4896 83.1534) (end 128.0034 83.1534) (width 0.75) (layer B.Cu) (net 17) (status 10))
 (segment (start 128.0034 83.1534) (end 129.5 84.65) (width 0.75) (layer B.Cu) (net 17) (status 20))
 (segment (start 127.04 90) (end 129 90) (width 0.75) (layer B.Cu) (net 25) (status 10))
 (segment (start 129 90) (end 129.5 89.5) (width 0.75) (layer B.Cu) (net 25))
 (segment (start 129.5 89.5) (end 129.5 87.35) (width 0.75) (layer B.Cu) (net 25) (status 20))
 (segment (start 129.5 89.5) (end 129.5 87.35) (width 0.5) (layer B.Cu) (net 25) (status 20))
 (segment (start 129 90) (end 129.5 89.5) (width 0.5) (layer B.Cu) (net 25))
 (segment (start 129.54 87.39) (end 129.5 87.35) (width 0.75) (layer B.Cu) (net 25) (status 30))
 (segment (start 125.4896 71.1646) (end 123.0146 71.1646) (width 1) (layer B.Cu) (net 11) (status 30))
 (segment (start 123.0146 71.1646) (end 122.85 71) (width 1) (layer B.Cu) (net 11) (status 30))
 (segment (start 125.4896 75.1778) (end 123.5278 75.1778) (width 1) (layer B.Cu) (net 13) (status 10))
 (segment (start 123.5278 75.1778) (end 122.85 74.5) (width 1) (layer B.Cu) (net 13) (status 20))
 (segment (start 119.54 93.81) (end 119.94 93.81) (width 1) (layer F.Cu) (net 22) (status 30))
 (segment (start 119.94 93.81) (end 121.25 92.5) (width 1) (layer F.Cu) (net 22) (status 10))
 (segment (start 119.94 93.81) (end 121.25 92.5) (width 0.75) (layer F.Cu) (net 22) (status 10))
 (segment (start 119.54 86.19) (end 119.54 93.81) (width 0.75) (layer F.Cu) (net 22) (status 30))
 (segment (start 119.35 89) (end 119.35 86.38) (width 0.75) (layer B.Cu) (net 22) (status 30))
 (segment (start 119.35 86.38) (end 119.54 86.19) (width 0.75) (layer B.Cu) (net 22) (status 30))
 (segment (start 119.94 93.81) (end 121.25 92.5) (width 0.5) (layer F.Cu) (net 22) (status 10))
 (segment (start 121.25 92.5) (end 122 91.75) (width 0.5) (layer F.Cu) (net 22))
 (segment (start 122 91.75) (end 128.65 91.75) (width 0.5) (layer F.Cu) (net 22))
 (segment (start 135 89.25) (end 135.5 89.75) (width 1) (layer B.Cu) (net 22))
 (segment (start 135.5 89.75) (end 135.25 89.5) (width 1) (layer F.Cu) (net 22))
 (via (at 135.5 89.75) (size 1.2) (drill 0.8) (layers F.Cu B.Cu) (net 22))
 (segment (start 135.25 89.5) (end 130.9 89.5) (width 0.5) (layer F.Cu) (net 22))
 (segment (start 130.9 89.5) (end 128.65 91.75) (width 0.5) (layer F.Cu) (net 22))
 (segment (start 133 79.5) (end 133 87.25) (width 0.5) (layer B.Cu) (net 22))
 (segment (start 133 87.25) (end 135 89.25) (width 0.5) (layer B.Cu) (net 22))
 (segment (start 133.309 79.191) (end 133 79.5) (width 0.5) (layer B.Cu) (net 22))
 (segment (start 137 79.191) (end 133.309 79.191) (width 0.5) (layer B.Cu) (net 22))
 (segment (start 139.5104 79.191) (end 137 79.191) (width 1) (layer B.Cu) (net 22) (status 10))
 (segment (start 137.35 81) (end 139.3382 81) (width 0.75) (layer B.Cu) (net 23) (status 30))
 (segment (start 139.3382 81) (end 139.5104 81.1722) (width 0.75) (layer B.Cu) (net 23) (status 30))
 (segment (start 139.3382 81) (end 139.5104 81.1722) (width 0.5) (layer B.Cu) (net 23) (status 30))
 (segment (start 139.3382 81) (end 139.5104 81.1722) (width 0.75) (layer B.Cu) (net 23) (status 30))
 (segment (start 137 83.65) (end 139.0392 83.65) (width 0.75) (layer B.Cu) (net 24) (status 30))
 (segment (start 139.0392 83.65) (end 139.5104 83.1788) (width 0.75) (layer B.Cu) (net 24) (status 30)))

